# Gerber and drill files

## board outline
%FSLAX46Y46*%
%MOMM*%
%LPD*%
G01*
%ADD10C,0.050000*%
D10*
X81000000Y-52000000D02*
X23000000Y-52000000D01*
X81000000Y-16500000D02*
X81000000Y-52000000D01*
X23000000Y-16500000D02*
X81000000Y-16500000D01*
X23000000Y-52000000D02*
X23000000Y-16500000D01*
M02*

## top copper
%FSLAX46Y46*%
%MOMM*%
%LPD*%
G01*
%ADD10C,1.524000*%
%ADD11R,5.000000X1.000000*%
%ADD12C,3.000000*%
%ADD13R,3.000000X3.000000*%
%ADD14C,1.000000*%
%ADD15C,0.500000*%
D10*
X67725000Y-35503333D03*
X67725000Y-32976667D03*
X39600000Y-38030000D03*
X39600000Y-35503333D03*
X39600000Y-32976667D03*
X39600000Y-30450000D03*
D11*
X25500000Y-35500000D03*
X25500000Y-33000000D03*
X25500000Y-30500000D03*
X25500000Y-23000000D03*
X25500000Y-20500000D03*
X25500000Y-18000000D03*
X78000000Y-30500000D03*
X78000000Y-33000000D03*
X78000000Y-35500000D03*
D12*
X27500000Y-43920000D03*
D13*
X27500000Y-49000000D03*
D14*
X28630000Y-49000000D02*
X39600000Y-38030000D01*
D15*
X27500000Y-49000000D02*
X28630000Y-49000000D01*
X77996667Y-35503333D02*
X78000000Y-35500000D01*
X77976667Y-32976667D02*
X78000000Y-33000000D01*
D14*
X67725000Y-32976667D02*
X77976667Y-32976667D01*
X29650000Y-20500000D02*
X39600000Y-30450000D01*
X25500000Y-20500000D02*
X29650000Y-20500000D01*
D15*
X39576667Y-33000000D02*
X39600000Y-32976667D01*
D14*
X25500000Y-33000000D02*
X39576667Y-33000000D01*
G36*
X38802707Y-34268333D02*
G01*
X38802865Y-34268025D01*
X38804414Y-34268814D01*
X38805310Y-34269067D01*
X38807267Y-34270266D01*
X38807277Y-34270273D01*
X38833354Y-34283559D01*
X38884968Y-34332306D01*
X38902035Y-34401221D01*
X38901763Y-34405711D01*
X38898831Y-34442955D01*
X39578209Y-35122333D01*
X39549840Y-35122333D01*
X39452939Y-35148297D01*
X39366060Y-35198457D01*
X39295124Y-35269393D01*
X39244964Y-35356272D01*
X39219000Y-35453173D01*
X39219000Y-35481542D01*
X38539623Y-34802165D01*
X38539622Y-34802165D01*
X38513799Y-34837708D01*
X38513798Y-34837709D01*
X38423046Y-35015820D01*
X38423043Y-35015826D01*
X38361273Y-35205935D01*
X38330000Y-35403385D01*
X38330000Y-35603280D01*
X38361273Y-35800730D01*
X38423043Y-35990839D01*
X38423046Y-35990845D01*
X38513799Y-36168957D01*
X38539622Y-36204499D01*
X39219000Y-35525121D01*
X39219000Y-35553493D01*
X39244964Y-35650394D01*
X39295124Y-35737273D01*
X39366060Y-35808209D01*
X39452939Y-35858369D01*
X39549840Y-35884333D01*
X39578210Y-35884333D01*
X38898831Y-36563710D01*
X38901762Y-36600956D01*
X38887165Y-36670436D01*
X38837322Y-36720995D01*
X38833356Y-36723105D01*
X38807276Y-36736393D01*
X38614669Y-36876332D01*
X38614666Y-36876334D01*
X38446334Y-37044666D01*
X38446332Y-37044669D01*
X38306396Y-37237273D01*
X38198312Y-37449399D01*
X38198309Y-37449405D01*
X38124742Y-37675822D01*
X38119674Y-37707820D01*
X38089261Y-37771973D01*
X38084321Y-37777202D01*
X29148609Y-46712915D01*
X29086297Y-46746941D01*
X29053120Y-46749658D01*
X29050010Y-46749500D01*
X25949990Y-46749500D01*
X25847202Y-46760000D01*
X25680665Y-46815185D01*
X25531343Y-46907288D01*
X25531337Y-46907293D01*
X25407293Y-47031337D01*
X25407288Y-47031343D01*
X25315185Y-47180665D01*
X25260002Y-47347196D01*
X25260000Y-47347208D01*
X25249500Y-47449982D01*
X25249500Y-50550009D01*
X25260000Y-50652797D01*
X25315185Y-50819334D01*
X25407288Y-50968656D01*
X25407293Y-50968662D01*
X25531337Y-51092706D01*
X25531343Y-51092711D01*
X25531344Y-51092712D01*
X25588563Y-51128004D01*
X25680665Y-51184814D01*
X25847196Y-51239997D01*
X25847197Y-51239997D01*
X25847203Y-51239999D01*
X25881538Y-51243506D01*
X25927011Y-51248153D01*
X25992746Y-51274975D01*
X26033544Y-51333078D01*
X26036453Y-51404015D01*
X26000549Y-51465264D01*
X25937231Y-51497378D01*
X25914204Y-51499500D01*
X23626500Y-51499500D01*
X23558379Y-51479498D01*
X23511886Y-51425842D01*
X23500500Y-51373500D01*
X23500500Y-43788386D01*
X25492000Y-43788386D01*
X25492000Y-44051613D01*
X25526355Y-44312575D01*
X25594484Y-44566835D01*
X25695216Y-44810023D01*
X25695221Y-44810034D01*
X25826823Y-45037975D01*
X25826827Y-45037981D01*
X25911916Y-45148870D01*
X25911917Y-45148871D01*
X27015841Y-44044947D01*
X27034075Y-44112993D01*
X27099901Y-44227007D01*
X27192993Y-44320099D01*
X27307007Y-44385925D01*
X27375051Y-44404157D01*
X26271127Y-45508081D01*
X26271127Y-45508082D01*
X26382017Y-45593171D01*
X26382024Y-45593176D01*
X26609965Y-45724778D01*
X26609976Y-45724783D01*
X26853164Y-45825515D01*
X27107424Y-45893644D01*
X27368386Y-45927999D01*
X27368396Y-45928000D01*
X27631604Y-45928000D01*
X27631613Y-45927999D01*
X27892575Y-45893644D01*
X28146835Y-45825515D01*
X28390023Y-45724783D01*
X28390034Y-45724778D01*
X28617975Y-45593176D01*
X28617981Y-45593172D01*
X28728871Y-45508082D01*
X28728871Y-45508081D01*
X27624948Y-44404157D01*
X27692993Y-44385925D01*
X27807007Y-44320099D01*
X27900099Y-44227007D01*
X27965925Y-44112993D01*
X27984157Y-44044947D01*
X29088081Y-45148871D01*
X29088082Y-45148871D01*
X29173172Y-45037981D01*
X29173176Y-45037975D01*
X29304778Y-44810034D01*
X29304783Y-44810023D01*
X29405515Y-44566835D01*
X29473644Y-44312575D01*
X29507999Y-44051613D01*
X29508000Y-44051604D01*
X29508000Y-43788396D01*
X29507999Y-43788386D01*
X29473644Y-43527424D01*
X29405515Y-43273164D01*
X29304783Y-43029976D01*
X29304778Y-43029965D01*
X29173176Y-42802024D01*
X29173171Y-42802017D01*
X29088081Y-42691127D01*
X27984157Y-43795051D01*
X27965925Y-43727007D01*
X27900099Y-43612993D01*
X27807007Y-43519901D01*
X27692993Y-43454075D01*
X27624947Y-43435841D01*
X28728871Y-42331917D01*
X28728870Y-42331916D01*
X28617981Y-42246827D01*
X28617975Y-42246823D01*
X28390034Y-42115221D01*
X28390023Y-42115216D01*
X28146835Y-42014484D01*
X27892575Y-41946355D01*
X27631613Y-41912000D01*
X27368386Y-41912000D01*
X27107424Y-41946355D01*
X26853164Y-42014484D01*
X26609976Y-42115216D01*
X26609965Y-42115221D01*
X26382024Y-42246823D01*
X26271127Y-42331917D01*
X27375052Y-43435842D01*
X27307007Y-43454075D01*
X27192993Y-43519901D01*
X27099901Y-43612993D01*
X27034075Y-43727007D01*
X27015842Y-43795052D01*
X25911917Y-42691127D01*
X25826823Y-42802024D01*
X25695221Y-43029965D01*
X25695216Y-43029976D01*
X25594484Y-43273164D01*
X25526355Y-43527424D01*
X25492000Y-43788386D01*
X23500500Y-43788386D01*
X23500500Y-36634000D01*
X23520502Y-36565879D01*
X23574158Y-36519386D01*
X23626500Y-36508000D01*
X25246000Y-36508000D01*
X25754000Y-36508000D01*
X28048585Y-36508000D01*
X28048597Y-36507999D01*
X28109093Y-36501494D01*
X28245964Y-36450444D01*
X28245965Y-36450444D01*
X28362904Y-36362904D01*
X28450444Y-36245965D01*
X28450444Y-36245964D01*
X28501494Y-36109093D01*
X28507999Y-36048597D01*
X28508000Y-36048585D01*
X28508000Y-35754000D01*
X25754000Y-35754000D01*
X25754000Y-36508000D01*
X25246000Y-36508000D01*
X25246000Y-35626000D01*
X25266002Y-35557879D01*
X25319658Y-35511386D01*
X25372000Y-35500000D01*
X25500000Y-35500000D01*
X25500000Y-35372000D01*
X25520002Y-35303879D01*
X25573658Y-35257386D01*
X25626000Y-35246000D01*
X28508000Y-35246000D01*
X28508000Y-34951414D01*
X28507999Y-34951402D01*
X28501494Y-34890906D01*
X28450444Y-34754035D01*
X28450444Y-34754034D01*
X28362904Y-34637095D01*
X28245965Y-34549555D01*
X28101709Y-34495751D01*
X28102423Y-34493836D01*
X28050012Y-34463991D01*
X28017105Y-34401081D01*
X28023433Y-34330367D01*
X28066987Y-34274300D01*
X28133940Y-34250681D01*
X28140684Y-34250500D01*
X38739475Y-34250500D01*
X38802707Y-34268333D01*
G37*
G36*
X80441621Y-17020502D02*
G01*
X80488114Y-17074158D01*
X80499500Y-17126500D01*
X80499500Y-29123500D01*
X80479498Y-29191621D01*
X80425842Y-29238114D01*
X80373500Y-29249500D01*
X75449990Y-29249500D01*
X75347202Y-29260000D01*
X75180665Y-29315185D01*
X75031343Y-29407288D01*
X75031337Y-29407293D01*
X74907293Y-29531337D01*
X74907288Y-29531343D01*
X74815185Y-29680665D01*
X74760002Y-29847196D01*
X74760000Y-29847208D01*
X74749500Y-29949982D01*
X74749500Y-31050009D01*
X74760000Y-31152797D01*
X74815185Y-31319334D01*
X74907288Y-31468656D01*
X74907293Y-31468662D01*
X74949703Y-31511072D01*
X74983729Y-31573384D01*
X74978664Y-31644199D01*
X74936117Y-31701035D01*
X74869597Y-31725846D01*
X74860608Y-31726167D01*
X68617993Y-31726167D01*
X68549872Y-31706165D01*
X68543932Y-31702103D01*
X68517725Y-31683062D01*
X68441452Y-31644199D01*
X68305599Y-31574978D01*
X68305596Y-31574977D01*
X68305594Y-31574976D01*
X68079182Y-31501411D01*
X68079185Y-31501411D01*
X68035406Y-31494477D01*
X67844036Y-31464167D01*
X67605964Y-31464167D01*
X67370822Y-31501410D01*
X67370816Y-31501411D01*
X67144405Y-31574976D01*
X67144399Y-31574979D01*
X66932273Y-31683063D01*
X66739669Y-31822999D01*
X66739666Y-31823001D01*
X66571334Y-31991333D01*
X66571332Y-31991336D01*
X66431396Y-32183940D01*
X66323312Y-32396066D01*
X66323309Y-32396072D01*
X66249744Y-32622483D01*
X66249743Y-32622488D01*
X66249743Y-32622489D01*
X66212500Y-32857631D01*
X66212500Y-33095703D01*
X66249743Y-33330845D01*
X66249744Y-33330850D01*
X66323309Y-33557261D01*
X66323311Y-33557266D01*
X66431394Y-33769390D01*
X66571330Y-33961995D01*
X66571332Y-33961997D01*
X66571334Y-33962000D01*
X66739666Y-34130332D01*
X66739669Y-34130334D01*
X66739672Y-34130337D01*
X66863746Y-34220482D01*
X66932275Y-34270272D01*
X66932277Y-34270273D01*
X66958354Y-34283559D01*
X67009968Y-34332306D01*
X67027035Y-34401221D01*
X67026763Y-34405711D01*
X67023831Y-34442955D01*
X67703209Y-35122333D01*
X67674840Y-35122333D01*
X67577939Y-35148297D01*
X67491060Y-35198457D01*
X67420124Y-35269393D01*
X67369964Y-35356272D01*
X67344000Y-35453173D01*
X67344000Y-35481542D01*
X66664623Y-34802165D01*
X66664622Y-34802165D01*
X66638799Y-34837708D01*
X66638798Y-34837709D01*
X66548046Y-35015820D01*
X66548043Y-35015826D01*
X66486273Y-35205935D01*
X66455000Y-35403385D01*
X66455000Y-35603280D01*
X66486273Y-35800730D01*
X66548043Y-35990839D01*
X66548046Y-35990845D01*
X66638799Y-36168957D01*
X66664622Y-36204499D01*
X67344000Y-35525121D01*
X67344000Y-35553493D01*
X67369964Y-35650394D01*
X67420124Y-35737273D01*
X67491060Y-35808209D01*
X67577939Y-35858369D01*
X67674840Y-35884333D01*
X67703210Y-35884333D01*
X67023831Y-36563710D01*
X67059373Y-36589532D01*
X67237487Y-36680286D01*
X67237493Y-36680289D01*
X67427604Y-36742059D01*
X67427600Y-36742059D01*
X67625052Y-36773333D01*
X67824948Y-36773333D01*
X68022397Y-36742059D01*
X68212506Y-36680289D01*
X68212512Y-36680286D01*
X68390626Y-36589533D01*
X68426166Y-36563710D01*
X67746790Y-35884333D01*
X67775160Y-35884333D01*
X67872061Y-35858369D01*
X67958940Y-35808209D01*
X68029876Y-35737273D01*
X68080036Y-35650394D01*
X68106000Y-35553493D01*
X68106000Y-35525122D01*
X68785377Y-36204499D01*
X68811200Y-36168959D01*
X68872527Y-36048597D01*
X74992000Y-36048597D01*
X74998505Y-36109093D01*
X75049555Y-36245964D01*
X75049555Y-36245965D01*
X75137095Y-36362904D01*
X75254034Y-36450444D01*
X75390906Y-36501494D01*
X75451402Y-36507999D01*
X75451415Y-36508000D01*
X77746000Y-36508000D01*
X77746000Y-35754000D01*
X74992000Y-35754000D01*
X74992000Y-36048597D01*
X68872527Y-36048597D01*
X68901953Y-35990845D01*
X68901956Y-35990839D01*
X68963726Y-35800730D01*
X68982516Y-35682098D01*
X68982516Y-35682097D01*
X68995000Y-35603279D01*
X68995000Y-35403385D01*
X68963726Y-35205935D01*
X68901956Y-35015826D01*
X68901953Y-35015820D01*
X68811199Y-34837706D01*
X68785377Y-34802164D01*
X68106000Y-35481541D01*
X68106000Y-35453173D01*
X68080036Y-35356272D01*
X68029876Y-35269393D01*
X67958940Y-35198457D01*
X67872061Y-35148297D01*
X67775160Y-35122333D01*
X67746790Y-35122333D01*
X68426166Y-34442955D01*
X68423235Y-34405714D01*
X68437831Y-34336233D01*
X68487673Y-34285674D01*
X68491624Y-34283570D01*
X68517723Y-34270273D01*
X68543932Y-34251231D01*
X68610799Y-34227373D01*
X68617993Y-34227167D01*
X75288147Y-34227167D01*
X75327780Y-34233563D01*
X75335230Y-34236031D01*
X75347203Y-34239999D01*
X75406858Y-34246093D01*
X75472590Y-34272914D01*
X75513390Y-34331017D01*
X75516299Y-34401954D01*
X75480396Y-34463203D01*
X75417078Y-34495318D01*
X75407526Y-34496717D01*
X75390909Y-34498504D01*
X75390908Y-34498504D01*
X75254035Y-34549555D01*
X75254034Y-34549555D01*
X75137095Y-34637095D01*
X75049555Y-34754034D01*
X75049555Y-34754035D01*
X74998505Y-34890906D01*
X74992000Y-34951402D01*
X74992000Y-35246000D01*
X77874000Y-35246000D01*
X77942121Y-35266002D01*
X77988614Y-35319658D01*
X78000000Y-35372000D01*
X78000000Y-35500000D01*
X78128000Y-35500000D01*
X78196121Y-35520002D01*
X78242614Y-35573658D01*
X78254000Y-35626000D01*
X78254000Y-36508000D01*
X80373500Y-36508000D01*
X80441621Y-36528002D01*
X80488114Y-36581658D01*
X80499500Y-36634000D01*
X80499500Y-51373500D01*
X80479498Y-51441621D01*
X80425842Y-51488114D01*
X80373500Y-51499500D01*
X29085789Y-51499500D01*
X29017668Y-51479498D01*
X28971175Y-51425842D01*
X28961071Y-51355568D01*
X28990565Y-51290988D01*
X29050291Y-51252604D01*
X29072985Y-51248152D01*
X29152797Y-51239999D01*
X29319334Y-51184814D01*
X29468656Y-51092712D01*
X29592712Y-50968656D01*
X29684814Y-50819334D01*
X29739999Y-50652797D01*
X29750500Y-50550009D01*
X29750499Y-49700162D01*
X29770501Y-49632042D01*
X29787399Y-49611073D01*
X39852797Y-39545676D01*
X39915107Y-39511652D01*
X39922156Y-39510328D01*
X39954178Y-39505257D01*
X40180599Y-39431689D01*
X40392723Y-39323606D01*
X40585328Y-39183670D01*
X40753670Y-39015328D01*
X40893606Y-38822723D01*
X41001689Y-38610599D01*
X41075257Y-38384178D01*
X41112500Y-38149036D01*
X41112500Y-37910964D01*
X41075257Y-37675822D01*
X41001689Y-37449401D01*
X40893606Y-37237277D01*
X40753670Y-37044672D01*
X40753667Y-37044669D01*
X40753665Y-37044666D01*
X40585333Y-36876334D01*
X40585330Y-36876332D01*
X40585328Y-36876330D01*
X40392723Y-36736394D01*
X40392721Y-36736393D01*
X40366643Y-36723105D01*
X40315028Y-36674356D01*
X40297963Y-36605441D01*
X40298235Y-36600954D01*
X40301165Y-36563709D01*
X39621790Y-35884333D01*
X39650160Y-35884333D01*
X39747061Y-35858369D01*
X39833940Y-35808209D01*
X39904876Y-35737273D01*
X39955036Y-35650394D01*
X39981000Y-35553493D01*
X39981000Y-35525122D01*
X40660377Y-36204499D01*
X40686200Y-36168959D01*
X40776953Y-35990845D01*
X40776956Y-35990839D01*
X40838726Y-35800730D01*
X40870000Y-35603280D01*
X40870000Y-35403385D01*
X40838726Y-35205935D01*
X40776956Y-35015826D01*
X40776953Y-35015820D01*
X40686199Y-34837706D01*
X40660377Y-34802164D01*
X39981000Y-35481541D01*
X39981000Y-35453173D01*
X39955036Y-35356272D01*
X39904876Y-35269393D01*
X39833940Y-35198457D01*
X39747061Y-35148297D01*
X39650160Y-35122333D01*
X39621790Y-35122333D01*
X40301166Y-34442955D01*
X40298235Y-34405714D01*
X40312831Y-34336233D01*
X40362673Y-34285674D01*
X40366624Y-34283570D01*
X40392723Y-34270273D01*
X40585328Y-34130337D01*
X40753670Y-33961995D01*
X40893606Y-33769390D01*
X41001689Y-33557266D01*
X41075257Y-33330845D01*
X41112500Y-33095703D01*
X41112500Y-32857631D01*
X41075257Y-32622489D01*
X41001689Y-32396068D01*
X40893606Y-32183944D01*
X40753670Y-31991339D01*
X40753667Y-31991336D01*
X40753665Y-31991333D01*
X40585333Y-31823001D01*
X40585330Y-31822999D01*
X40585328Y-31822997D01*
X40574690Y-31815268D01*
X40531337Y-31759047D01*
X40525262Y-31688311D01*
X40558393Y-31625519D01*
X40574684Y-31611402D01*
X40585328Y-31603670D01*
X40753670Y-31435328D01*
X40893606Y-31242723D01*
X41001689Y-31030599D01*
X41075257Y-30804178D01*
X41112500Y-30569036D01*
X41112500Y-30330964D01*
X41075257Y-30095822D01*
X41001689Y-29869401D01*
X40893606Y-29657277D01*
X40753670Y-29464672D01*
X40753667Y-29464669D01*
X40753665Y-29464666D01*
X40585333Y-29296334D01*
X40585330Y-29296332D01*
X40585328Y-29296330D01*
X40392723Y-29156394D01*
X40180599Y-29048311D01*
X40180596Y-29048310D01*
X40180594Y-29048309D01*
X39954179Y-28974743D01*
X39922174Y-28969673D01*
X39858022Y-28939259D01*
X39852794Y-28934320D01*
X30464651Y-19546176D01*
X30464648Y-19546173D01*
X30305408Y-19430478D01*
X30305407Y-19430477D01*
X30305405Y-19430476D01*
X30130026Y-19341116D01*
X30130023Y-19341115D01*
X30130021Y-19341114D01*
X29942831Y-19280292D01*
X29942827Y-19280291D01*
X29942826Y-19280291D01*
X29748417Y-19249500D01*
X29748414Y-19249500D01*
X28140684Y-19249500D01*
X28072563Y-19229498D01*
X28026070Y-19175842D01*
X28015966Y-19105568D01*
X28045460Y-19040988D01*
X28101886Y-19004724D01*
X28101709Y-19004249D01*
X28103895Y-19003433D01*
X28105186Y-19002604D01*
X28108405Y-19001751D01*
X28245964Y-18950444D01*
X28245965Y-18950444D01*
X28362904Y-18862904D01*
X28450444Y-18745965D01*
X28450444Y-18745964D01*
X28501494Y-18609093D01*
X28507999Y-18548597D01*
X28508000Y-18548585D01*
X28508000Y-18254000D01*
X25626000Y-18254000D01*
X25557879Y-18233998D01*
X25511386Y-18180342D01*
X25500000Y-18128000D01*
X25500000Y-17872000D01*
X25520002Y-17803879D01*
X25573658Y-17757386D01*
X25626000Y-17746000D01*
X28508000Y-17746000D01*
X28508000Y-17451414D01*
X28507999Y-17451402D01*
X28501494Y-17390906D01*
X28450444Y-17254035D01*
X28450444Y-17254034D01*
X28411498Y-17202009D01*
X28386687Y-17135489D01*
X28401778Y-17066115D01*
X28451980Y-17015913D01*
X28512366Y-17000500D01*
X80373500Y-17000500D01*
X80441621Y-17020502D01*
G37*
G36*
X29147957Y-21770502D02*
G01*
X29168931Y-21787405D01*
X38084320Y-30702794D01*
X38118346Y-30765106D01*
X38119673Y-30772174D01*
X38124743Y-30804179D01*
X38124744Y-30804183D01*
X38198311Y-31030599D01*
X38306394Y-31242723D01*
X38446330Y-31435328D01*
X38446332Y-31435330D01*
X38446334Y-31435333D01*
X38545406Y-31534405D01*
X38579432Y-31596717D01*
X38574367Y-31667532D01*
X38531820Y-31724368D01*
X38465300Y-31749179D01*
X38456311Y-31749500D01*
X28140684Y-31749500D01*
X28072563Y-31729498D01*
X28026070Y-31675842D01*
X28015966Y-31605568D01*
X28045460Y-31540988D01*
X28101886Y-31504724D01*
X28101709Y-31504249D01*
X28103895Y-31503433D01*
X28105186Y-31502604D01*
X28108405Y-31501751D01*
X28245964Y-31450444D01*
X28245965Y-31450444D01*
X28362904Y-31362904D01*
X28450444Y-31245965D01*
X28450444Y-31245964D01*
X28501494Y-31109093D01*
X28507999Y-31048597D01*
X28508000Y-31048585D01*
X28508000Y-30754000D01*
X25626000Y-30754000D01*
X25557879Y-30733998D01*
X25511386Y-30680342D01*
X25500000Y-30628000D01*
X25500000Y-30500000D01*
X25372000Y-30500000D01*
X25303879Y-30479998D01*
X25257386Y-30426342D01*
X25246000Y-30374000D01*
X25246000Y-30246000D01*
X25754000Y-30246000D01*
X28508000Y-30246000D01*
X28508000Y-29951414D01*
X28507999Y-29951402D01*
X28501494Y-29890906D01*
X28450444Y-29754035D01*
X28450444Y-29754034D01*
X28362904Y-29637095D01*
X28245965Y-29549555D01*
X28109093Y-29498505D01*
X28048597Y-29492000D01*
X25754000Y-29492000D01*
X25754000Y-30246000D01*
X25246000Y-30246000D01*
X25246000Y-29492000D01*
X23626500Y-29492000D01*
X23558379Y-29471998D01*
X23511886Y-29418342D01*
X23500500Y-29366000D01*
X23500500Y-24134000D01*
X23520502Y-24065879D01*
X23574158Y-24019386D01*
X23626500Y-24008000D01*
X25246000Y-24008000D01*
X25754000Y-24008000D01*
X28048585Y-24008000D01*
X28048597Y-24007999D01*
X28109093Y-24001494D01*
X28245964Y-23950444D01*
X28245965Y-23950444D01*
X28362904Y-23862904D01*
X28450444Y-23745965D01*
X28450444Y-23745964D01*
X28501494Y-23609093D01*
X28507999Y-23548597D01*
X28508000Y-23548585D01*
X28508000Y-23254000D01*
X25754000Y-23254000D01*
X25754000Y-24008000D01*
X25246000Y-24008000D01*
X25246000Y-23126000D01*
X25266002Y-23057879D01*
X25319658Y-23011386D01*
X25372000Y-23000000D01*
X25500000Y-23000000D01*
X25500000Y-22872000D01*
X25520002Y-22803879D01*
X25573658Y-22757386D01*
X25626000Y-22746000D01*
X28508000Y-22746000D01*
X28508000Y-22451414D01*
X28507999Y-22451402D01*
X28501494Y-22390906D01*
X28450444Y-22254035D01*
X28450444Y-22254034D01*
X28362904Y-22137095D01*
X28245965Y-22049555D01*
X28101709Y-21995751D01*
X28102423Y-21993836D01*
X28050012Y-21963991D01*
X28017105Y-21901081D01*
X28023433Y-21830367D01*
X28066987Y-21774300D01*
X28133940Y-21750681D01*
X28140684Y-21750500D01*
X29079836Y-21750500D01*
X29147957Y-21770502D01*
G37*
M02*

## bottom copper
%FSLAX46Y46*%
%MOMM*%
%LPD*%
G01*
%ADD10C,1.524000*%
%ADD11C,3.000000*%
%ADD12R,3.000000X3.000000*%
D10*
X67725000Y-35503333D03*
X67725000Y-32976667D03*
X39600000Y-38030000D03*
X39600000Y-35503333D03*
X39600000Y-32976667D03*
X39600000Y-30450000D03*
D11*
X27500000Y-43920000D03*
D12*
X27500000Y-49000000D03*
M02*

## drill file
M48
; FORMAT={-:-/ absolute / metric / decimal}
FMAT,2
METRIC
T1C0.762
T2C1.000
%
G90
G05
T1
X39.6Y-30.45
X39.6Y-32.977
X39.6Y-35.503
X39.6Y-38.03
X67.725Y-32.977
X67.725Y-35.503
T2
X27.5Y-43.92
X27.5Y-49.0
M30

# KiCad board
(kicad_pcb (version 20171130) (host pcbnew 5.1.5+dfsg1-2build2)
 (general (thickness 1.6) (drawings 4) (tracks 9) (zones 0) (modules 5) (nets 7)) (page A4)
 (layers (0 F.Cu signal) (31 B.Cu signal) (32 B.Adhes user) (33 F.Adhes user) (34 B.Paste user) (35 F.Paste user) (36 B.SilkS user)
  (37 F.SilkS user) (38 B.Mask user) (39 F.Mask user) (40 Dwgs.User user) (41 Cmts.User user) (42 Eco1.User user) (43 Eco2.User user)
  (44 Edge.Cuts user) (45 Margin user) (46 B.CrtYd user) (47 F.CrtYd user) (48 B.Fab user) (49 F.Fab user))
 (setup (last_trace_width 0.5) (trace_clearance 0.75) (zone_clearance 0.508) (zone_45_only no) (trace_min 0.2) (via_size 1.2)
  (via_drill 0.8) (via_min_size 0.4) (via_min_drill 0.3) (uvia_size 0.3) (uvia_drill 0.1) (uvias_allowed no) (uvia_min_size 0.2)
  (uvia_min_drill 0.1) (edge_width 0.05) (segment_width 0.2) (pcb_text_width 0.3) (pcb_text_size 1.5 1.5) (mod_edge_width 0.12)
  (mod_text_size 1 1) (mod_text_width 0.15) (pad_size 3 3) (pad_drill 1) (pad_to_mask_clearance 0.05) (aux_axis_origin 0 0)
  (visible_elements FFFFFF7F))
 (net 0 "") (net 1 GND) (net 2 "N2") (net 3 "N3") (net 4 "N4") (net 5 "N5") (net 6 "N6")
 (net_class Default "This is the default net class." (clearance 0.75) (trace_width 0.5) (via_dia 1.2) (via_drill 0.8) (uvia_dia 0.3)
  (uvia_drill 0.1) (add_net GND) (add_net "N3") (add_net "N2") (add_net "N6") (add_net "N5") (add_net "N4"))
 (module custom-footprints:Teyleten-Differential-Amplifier (layer F.Cu) (at 33 35.5 90)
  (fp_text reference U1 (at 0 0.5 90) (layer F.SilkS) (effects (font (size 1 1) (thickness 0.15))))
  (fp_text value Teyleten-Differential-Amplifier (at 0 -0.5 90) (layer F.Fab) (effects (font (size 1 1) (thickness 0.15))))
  (pad 6 thru_hole circle (at -0.003333 34.725) (size 1.524 1.524) (drill 0.762) (layers *.Cu *.Mask) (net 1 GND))
  (pad 5 thru_hole circle (at 2.523333 34.725 90) (size 1.524 1.524) (drill 0.762) (layers *.Cu *.Mask) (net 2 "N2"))
  (pad 4 thru_hole circle (at -2.53 6.6 180) (size 1.524 1.524) (drill 0.762) (layers *.Cu *.Mask) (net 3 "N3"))
  (pad 3 thru_hole circle (at -0.003333 6.6) (size 1.524 1.524) (drill 0.762) (layers *.Cu *.Mask) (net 1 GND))
  (pad 2 thru_hole circle (at 2.523333 6.6 90) (size 1.524 1.524) (drill 0.762) (layers *.Cu *.Mask) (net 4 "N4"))
  (pad 1 thru_hole circle (at 5.05 6.6 90) (size 1.524 1.524) (drill 0.762) (layers *.Cu *.Mask) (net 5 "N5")))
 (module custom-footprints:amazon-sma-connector (layer F.Cu) (at 22.5 27.5)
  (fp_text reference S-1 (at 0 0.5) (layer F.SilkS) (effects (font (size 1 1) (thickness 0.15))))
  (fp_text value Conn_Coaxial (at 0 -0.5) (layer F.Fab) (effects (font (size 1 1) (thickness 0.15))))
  (pad 2 connect rect (at 3 8) (size 5 1) (layers F.Cu F.Mask) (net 1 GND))
  (pad 1 connect rect (at 3 5.5) (size 5 1) (layers F.Cu F.Mask) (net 4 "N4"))
  (pad 2 connect rect (at 3 3) (size 5 1) (layers F.Cu F.Mask) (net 1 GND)))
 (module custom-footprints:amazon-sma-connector (layer F.Cu) (at 22.5 15)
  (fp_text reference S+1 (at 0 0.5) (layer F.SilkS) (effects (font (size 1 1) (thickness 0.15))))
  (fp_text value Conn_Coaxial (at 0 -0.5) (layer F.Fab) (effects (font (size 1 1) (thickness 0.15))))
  (pad 2 connect rect (at 3 8) (size 5 1) (layers F.Cu F.Mask) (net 1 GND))
  (pad 1 connect rect (at 3 5.5) (size 5 1) (layers F.Cu F.Mask) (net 5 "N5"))
  (pad 2 connect rect (at 3 3) (size 5 1) (layers F.Cu F.Mask) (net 1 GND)))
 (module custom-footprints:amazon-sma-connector (layer F.Cu) (at 81 38.5 180)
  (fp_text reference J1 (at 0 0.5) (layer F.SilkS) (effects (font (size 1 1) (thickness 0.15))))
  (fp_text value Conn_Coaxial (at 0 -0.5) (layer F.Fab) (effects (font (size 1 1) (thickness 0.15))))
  (pad 2 connect rect (at 3 8 180) (size 5 1) (layers F.Cu F.Mask) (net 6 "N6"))
  (pad 1 connect rect (at 3 5.5 180) (size 5 1) (layers F.Cu F.Mask) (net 2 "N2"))
  (pad 2 connect rect (at 3 3 180) (size 5 1) (layers F.Cu F.Mask) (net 1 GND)))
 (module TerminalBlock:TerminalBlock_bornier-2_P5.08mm (layer F.Cu) (at 27.5 49 90)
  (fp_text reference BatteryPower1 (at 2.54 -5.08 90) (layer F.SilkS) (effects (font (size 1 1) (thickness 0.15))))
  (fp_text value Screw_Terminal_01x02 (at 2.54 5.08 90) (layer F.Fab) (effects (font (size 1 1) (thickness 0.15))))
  (pad 2 thru_hole circle (at 5.08 0 90) (size 3 3) (drill 1) (layers *.Cu *.Mask) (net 1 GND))
  (pad 1 thru_hole rect (at 0 0 90) (size 3 3) (drill 1) (layers *.Cu *.Mask) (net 3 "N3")))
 (gr_line (start 81 52) (end 23 52) (layer Edge.Cuts) (width 0.05))
 (gr_line (start 81 16.5) (end 81 52) (layer Edge.Cuts) (width 0.05))
 (gr_line (start 23 16.5) (end 81 16.5) (layer Edge.Cuts) (width 0.05))
 (gr_line (start 23 52) (end 23 16.5) (layer Edge.Cuts) (width 0.05))
 (segment (start 28.63 49) (end 39.6 38.03) (width 1) (layer F.Cu) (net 3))
 (segment (start 27.5 49) (end 28.63 49) (width 0.5) (layer F.Cu) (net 3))
 (segment (start 77.996667 35.503333) (end 78 35.5) (width 0.5) (layer F.Cu) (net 1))
 (segment (start 77.976667 32.976667) (end 78 33) (width 0.5) (layer F.Cu) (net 2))
 (segment (start 67.725 32.976667) (end 77.976667 32.976667) (width 1) (layer F.Cu) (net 2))
 (segment (start 29.65 20.5) (end 39.6 30.45) (width 1) (layer F.Cu) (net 5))
 (segment (start 25.5 20.5) (end 29.65 20.5) (width 1) (layer F.Cu) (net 5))
 (segment (start 39.576667 33) (end 39.6 32.976667) (width 0.5) (layer F.Cu) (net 4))
 (segment (start 25.5 33) (end 39.576667 33) (width 1) (layer F.Cu) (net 4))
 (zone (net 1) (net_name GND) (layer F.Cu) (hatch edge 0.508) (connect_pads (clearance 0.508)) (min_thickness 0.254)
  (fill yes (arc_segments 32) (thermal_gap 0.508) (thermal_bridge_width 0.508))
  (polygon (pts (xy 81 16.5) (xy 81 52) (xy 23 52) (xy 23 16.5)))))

